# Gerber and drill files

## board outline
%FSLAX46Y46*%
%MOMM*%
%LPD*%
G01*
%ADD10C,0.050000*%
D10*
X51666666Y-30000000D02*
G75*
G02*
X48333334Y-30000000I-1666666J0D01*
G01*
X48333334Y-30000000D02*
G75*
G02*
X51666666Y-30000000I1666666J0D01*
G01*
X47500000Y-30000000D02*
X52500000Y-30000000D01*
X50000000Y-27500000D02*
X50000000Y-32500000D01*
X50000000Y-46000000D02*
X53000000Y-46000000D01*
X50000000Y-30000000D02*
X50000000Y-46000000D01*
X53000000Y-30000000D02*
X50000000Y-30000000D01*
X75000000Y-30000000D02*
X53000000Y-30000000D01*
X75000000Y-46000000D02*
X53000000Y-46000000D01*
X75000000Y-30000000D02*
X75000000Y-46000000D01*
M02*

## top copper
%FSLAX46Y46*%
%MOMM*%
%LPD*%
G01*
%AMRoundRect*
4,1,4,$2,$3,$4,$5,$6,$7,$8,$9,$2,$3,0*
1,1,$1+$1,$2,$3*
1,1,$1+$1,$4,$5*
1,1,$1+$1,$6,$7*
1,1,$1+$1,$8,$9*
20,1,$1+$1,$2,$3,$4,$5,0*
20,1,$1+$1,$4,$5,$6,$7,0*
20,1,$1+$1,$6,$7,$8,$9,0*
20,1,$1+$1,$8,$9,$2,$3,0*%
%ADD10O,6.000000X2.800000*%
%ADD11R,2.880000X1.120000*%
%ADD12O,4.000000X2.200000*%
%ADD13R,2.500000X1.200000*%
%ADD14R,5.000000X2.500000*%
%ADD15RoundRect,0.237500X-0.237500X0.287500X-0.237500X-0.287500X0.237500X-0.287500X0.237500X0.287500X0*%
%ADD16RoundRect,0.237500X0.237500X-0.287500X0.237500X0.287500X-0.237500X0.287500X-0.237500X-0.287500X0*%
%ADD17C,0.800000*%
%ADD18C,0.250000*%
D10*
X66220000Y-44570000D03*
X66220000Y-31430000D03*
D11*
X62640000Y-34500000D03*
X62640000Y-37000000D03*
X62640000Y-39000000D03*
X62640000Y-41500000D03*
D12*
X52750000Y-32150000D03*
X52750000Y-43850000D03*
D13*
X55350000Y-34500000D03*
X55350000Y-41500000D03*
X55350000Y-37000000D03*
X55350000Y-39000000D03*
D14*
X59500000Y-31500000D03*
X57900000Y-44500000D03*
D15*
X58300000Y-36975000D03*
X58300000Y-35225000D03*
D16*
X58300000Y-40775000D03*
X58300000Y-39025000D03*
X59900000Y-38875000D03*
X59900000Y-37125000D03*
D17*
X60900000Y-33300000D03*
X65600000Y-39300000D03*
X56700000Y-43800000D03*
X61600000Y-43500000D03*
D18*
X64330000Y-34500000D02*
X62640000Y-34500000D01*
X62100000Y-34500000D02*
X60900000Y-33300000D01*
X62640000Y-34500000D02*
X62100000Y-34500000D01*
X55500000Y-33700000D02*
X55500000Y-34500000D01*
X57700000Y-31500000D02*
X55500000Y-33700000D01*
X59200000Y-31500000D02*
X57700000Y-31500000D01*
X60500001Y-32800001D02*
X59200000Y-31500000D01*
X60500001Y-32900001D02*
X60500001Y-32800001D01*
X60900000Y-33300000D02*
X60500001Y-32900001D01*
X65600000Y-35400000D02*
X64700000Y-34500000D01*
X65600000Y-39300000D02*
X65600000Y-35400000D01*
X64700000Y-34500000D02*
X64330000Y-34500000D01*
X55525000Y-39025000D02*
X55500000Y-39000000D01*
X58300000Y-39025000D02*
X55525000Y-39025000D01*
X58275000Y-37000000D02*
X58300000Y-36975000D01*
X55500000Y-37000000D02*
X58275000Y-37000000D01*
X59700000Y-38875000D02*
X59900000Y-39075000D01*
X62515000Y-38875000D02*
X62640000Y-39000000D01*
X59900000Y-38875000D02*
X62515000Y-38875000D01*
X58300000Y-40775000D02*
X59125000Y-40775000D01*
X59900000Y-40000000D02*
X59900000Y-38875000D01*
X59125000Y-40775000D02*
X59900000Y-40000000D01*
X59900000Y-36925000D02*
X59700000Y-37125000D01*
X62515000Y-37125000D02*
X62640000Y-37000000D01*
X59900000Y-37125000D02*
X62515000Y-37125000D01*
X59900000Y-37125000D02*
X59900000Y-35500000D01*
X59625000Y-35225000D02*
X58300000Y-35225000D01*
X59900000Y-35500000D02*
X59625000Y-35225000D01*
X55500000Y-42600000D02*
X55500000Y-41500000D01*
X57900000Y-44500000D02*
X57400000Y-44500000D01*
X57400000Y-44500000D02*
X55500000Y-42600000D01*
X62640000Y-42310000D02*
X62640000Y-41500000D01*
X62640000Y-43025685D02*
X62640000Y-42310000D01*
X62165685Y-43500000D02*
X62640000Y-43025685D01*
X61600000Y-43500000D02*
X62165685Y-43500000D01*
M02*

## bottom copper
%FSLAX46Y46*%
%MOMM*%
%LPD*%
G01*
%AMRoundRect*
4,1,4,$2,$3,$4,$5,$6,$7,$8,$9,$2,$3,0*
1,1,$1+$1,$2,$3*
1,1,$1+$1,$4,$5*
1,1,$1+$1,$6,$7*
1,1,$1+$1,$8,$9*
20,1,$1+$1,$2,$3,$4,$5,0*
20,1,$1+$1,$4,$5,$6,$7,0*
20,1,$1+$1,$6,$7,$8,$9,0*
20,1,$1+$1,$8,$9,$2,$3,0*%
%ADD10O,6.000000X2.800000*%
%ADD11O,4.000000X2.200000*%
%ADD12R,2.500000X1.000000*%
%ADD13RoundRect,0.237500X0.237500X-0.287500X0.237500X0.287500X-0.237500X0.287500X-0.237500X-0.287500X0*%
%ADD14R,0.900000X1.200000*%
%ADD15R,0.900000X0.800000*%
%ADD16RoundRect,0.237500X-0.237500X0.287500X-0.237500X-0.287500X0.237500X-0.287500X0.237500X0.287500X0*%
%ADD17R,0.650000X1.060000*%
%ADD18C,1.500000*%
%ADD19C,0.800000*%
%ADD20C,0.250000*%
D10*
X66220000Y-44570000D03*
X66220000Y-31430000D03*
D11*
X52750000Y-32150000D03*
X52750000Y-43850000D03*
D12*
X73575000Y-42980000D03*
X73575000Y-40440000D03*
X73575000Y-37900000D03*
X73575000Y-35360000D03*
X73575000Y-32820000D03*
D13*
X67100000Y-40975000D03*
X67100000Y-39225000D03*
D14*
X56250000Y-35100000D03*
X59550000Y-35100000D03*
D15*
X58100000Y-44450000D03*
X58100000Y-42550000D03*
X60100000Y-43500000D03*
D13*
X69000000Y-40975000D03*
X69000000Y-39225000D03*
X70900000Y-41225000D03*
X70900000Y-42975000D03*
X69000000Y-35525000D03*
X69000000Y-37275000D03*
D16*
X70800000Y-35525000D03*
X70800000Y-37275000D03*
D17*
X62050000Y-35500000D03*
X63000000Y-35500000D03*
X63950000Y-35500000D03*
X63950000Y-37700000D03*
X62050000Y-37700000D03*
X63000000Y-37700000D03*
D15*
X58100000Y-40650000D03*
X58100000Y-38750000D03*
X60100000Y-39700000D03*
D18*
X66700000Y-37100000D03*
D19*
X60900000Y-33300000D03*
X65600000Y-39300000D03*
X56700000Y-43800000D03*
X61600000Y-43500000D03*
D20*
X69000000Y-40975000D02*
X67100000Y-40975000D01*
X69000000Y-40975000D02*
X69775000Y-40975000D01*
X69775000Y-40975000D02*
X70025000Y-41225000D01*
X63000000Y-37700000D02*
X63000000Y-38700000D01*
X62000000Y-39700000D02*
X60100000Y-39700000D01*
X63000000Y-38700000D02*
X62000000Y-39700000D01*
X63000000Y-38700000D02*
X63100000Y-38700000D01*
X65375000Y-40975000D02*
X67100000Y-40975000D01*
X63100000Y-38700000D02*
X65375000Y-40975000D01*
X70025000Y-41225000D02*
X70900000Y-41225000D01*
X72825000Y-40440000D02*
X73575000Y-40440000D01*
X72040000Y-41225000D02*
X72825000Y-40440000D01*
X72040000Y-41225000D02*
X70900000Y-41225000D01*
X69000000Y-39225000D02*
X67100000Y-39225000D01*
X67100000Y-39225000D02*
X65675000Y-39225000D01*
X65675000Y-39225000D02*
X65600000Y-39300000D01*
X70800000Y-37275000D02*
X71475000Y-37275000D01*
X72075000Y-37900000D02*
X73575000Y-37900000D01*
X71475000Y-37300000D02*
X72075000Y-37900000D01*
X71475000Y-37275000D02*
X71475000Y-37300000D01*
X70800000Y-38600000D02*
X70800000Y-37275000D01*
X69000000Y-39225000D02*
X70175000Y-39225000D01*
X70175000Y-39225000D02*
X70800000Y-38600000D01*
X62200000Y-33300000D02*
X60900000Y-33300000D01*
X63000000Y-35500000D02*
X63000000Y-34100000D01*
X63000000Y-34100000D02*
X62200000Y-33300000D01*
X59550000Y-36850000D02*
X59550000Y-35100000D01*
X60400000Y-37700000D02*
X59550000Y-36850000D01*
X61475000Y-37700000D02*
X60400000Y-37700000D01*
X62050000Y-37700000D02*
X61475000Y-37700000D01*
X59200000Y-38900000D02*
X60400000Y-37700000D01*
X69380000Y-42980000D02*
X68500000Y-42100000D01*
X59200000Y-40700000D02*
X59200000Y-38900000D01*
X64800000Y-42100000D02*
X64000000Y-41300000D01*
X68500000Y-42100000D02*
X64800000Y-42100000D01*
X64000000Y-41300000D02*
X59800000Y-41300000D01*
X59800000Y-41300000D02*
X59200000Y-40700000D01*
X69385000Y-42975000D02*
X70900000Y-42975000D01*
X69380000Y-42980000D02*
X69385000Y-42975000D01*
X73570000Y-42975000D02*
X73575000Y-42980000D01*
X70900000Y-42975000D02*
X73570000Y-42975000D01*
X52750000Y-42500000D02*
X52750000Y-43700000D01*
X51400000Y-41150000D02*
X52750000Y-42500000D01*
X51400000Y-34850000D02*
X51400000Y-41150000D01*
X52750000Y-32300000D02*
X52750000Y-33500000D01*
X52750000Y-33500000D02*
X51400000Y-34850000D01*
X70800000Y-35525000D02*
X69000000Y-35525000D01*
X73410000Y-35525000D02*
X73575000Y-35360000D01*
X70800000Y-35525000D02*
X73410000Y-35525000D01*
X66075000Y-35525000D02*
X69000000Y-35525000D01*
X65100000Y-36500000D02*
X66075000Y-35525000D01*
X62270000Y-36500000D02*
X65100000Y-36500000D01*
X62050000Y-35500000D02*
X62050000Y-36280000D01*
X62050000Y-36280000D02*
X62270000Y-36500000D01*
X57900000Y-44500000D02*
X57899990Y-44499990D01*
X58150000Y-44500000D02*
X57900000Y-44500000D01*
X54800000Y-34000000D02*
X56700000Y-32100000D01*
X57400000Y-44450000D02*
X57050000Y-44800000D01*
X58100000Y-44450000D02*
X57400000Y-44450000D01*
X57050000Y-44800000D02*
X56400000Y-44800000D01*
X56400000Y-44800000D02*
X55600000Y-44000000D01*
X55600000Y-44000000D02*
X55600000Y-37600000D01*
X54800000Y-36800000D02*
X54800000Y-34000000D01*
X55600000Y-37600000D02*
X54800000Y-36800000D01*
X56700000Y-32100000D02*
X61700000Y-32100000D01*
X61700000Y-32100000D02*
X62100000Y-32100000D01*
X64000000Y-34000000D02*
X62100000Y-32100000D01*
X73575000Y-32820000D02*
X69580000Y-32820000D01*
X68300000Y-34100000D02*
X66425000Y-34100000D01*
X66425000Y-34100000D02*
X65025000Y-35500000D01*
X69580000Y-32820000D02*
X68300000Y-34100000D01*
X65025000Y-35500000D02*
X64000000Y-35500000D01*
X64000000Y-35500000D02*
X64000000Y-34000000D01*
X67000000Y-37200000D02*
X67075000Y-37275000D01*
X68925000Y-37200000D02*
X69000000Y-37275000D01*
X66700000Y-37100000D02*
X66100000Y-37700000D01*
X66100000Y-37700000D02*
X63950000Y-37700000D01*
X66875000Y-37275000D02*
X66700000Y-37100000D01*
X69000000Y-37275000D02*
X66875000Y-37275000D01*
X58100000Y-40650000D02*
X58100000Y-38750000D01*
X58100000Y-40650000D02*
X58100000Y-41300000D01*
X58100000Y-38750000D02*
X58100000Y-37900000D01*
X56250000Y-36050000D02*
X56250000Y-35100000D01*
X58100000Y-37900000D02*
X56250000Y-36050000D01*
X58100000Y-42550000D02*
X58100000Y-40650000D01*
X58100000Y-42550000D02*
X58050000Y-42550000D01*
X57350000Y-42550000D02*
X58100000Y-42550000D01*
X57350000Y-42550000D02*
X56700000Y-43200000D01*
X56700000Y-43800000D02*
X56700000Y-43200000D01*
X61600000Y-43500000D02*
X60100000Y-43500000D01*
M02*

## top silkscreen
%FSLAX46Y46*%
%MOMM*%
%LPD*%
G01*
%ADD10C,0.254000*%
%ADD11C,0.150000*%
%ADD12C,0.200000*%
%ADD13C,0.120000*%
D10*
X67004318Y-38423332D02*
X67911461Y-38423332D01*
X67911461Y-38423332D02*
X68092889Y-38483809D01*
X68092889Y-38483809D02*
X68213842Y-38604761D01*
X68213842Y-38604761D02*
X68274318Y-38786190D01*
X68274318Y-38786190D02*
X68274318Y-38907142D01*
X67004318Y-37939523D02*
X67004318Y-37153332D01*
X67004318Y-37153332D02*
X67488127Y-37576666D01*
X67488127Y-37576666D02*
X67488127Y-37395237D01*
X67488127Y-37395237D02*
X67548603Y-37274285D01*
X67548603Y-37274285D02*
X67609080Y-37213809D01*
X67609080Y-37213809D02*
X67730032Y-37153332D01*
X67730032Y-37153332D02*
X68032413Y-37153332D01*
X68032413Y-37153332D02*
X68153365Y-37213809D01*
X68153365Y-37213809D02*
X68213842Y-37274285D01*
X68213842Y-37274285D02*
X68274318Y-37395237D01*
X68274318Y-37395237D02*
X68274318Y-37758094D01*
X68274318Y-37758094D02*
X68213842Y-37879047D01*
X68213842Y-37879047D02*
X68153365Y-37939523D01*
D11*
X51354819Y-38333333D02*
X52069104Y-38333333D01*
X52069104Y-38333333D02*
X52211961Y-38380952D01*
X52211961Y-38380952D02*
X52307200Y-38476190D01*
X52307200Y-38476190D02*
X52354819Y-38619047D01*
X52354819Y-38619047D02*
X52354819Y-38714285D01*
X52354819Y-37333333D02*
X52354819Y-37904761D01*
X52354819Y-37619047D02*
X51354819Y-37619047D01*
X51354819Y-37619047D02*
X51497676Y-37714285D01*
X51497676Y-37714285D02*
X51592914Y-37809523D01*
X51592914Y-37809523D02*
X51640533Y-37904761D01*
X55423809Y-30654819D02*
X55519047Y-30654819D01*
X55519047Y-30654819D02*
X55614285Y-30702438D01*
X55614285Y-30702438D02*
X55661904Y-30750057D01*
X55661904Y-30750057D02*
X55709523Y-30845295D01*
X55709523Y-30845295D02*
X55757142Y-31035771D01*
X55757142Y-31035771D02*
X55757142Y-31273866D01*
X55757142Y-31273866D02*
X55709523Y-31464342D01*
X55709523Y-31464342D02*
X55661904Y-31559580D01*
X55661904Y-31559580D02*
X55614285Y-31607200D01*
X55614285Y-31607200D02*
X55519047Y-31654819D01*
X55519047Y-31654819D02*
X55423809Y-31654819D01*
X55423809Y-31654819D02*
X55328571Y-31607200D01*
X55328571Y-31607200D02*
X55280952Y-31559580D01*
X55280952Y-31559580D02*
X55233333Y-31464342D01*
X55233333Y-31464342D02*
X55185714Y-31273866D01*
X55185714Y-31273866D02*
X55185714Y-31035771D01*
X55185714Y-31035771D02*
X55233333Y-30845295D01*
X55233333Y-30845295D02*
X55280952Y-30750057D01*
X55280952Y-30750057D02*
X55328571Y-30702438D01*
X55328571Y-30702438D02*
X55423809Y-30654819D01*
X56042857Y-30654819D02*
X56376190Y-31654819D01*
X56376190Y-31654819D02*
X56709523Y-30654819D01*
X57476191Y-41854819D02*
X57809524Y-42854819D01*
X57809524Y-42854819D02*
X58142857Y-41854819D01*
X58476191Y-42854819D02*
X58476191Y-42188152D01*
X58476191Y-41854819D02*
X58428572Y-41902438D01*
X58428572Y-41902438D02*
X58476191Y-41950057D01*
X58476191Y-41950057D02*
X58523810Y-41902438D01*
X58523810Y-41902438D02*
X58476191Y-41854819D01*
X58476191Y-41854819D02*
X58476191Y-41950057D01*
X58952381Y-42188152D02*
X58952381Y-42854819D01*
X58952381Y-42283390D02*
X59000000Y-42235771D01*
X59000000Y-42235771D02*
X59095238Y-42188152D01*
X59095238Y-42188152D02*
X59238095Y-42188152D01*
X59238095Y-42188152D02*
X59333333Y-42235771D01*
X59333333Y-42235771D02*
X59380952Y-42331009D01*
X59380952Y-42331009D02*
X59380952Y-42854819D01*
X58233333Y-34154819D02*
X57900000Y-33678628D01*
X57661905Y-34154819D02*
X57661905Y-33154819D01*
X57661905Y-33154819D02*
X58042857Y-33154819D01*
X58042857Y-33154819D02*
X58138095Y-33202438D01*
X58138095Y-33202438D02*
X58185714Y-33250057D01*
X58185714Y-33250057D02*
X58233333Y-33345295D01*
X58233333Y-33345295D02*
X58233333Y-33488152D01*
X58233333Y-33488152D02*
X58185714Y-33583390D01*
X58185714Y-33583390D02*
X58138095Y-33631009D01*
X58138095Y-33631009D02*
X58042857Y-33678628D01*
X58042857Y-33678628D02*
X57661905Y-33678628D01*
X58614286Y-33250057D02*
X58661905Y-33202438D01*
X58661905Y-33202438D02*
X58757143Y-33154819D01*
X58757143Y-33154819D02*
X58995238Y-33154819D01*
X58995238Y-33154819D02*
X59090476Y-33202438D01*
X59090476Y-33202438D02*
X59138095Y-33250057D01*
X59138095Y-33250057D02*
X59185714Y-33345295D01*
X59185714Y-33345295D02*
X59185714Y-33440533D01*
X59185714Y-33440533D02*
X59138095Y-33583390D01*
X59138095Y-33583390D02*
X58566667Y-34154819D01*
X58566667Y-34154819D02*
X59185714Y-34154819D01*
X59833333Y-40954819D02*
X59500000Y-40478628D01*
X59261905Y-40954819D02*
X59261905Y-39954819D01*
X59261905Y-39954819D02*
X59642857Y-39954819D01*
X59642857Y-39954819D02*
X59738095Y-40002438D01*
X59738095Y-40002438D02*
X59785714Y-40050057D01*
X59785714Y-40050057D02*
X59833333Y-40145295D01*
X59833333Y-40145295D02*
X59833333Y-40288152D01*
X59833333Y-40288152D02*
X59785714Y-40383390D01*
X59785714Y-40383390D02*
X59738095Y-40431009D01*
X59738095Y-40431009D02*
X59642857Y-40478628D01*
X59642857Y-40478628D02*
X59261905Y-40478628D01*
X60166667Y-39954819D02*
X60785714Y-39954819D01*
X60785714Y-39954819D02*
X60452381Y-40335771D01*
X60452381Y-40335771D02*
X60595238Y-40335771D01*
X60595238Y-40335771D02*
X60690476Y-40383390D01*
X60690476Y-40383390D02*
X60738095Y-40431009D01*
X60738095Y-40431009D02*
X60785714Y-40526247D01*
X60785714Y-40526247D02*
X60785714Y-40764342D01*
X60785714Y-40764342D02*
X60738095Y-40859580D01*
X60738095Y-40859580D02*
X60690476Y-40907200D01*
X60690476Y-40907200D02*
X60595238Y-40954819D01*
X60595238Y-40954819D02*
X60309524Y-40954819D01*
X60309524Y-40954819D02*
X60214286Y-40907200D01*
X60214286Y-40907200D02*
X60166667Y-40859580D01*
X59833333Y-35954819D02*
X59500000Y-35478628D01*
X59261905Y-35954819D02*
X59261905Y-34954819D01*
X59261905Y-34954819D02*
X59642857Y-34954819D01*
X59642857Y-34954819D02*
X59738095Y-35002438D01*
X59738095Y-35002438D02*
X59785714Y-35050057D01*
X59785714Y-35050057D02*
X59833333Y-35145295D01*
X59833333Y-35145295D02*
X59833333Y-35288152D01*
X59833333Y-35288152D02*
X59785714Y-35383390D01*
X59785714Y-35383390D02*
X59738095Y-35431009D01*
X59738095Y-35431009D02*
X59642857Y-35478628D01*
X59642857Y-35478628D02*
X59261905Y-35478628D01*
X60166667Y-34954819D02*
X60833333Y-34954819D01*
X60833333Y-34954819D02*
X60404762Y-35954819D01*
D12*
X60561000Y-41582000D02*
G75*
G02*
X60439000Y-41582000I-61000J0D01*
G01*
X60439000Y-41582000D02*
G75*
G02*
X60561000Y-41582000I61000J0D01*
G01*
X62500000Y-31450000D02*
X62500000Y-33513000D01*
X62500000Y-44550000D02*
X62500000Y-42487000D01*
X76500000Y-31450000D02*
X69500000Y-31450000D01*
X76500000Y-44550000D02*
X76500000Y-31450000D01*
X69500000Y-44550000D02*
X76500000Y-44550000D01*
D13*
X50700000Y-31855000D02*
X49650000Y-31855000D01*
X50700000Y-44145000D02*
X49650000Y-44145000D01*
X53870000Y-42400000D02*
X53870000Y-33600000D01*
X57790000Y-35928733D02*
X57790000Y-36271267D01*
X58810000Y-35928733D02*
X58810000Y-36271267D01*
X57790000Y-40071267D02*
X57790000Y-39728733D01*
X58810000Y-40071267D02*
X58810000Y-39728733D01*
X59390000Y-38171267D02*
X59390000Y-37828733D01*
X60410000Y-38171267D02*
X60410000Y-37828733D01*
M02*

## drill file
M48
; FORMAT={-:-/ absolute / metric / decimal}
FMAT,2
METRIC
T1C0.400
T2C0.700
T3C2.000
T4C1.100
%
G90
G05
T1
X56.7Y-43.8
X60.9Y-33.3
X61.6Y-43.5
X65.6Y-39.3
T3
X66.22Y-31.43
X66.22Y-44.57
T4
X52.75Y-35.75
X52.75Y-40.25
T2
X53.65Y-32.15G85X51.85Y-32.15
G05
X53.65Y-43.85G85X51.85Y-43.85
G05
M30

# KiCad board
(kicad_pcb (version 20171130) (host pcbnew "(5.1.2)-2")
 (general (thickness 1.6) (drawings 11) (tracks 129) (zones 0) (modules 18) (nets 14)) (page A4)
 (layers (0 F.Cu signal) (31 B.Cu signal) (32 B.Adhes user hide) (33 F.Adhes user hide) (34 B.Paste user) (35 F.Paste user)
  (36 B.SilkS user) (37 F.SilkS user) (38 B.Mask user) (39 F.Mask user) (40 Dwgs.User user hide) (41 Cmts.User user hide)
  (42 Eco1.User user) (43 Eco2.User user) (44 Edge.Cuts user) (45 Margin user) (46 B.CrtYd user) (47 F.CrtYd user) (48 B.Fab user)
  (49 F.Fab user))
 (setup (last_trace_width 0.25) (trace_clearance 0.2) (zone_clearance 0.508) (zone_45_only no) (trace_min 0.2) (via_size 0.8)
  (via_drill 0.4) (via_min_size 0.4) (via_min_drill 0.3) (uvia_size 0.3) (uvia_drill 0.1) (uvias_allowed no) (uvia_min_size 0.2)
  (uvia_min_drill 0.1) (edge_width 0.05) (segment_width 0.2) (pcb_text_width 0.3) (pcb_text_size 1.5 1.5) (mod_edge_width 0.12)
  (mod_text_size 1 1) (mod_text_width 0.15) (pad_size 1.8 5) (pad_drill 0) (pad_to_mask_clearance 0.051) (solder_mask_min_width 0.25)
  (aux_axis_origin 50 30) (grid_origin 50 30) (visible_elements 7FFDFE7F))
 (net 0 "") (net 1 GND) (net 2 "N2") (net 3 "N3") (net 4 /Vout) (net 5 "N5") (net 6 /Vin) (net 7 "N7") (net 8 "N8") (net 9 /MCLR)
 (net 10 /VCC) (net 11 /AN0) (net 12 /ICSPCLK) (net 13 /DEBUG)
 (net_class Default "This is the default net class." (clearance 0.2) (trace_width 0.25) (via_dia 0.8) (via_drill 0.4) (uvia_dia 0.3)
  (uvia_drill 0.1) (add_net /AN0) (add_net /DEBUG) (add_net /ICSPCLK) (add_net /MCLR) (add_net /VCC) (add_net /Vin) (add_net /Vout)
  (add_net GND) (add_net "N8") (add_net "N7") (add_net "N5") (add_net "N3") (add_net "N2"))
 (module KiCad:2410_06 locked (layer F.Cu) (at 76.5 38 90)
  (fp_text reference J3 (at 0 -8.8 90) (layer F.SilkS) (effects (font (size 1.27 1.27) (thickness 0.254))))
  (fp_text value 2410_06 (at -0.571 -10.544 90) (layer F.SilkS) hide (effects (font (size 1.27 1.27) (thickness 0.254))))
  (fp_circle (center -3.582 -16) (end -3.582 -15.939) (layer F.SilkS) (width 0.2))
  (fp_line (start 6.55 -14) (end 4.487 -14) (layer F.SilkS) (width 0.2))
  (fp_line (start -6.55 -14) (end -4.487 -14) (layer F.SilkS) (width 0.2))
  (fp_line (start 6.55 0) (end 6.55 -7) (layer F.SilkS) (width 0.2))
  (fp_line (start -6.55 0) (end 6.55 0) (layer F.SilkS) (width 0.2))
  (fp_line (start -6.55 -7) (end -6.55 0) (layer F.SilkS) (width 0.2))
  (pad 6 thru_hole oval (at -6.57 -10.28 90) (size 2.8 6) (drill 2) (layers *.Cu *.Mask))
  (pad 5 thru_hole oval (at 6.57 -10.28 90) (size 2.8 6) (drill 2) (layers *.Cu *.Mask))
  (pad 4 smd rect (at 3.5 -13.86 90) (size 1.12 2.88) (layers F.Cu F.Paste F.Mask) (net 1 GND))
  (pad 3 smd rect (at 1 -13.86 90) (size 1.12 2.88) (layers F.Cu F.Paste F.Mask) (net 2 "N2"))
  (pad 2 smd rect (at -1 -13.86 90) (size 1.12 2.88) (layers F.Cu F.Paste F.Mask) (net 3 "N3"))
  (pad 1 smd rect (at -3.5 -13.86 90) (size 1.12 2.88) (layers F.Cu F.Paste F.Mask) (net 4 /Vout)))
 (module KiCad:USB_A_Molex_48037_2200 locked (layer F.Cu) (at 45.85 38 180)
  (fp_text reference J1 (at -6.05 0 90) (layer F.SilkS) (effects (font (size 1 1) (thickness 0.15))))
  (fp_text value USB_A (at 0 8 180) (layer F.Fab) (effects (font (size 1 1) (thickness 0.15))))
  (fp_line (start -4.85 6.145) (end -3.8 6.145) (layer F.SilkS) (width 0.12))
  (fp_line (start -4.85 -6.145) (end -3.8 -6.145) (layer F.SilkS) (width 0.12))
  (fp_line (start -8.02 -4.4) (end -8.02 4.4) (layer F.SilkS) (width 0.12))
  (pad "" np_thru_hole circle (at -6.9 2.25 180) (size 1.1 1.1) (drill 1.1) (layers *.Cu *.Mask))
  (pad "" np_thru_hole circle (at -6.9 -2.25 180) (size 1.1 1.1) (drill 1.1) (layers *.Cu *.Mask))
  (pad 5 thru_hole oval (at -6.9 5.85 180) (size 4 2.2) (drill oval 2.5 0.7) (layers *.Cu *.Mask) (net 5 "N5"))
  (pad 5 thru_hole oval (at -6.9 -5.85 180) (size 4 2.2) (drill oval 2.5 0.7) (layers *.Cu *.Mask) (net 5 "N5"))
  (pad 4 smd rect (at -9.5 3.5 180) (size 2.5 1.2) (layers F.Cu F.Paste F.Mask) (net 1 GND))
  (pad 1 smd rect (at -9.5 -3.5 180) (size 2.5 1.2) (layers F.Cu F.Paste F.Mask) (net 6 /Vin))
  (pad 3 smd rect (at -9.5 1 180) (size 2.5 1.2) (layers F.Cu F.Paste F.Mask) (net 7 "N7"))
  (pad 2 smd rect (at -9.5 -1 180) (size 2.5 1.2) (layers F.Cu F.Paste F.Mask) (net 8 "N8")))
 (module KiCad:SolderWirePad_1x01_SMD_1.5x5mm (layer F.Cu) (at 59.5 31.5 90)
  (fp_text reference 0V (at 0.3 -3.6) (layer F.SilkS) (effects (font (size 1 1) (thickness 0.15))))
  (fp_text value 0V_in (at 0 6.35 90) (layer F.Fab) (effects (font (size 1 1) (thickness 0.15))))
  (pad 1 smd rect (at 0 0 90) (size 2.5 5) (layers F.Cu F.Paste F.Mask) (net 1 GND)))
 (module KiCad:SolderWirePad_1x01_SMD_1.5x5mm (layer F.Cu) (at 57.9 44.5 270)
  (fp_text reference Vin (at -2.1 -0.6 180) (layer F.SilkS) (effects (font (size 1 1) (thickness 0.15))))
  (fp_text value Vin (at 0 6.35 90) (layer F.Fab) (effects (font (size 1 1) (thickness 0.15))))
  (pad 1 smd rect (at 0 0 270) (size 2.5 5) (layers F.Cu F.Paste F.Mask) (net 6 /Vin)))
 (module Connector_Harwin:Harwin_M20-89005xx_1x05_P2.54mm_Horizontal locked (layer B.Cu) (at 79.1 37.9)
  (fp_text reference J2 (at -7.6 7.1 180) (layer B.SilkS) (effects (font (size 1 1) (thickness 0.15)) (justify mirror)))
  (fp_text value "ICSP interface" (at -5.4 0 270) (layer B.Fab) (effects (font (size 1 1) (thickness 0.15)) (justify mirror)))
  (pad 1 smd rect (at -5.525 5.08) (size 2.5 1) (layers B.Cu B.Paste B.Mask) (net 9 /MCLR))
  (pad 2 smd rect (at -5.525 2.54) (size 2.5 1) (layers B.Cu B.Paste B.Mask) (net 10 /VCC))
  (pad 3 smd rect (at -5.525 0) (size 2.5 1) (layers B.Cu B.Paste B.Mask) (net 1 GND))
  (pad 4 smd rect (at -5.525 -2.54) (size 2.5 1) (layers B.Cu B.Paste B.Mask) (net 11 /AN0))
  (pad 5 smd rect (at -5.525 -5.08) (size 2.5 1) (layers B.Cu B.Paste B.Mask) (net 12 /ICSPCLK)))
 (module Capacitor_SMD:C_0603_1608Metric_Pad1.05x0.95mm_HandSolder (layer B.Cu) (at 67.1 40.1 90)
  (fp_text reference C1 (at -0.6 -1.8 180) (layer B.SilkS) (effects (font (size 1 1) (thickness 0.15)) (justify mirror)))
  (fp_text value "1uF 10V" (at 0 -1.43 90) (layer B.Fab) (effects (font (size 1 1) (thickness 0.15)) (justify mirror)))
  (pad 1 smd roundrect (at -0.875 0 90) (size 1.05 0.95) (layers B.Cu B.Paste B.Mask) (roundrect_rratio 0.25) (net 10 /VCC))
  (pad 2 smd roundrect (at 0.875 0 90) (size 1.05 0.95) (layers B.Cu B.Paste B.Mask) (roundrect_rratio 0.25) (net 1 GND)))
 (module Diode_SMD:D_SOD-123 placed (layer B.Cu) (at 57.9 35.1)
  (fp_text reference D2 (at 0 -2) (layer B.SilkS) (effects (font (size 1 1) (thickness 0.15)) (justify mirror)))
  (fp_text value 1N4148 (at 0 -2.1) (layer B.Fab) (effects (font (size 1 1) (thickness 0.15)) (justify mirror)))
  (pad 1 smd rect (at -1.65 0) (size 0.9 1.2) (layers B.Cu B.Paste B.Mask) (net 6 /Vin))
  (pad 2 smd rect (at 1.65 0) (size 0.9 1.2) (layers B.Cu B.Paste B.Mask) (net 9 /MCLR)))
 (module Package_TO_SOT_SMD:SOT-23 (layer B.Cu) (at 59.1 43.5)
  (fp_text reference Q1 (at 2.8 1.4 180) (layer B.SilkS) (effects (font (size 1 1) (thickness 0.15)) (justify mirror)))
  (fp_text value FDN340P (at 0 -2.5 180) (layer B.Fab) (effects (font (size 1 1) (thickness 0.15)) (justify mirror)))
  (pad 1 smd rect (at -1 0.95) (size 0.9 0.8) (layers B.Cu B.Paste B.Mask) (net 12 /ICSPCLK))
  (pad 2 smd rect (at -1 -0.95) (size 0.9 0.8) (layers B.Cu B.Paste B.Mask) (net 6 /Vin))
  (pad 3 smd rect (at 1 0) (size 0.9 0.8) (layers B.Cu B.Paste B.Mask) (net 4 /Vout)))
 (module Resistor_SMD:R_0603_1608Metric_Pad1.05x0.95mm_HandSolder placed (layer B.Cu) (at 69 40.1 90)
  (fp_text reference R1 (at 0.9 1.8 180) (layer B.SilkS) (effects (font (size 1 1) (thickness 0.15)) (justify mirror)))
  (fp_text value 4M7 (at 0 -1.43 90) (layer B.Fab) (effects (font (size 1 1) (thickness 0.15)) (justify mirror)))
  (pad 1 smd roundrect (at -0.875 0 90) (size 1.05 0.95) (layers B.Cu B.Paste B.Mask) (roundrect_rratio 0.25) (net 10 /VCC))
  (pad 2 smd roundrect (at 0.875 0 90) (size 1.05 0.95) (layers B.Cu B.Paste B.Mask) (roundrect_rratio 0.25) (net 1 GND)))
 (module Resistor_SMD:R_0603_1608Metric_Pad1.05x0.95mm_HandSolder (layer F.Cu) (at 58.3 36.1 270)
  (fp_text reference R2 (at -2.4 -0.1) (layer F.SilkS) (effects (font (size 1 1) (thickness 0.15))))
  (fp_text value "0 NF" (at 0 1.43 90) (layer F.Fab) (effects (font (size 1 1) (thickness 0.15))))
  (fp_line (start -0.171267 0.51) (end 0.171267 0.51) (layer F.SilkS) (width 0.12))
  (fp_line (start -0.171267 -0.51) (end 0.171267 -0.51) (layer F.SilkS) (width 0.12))
  (pad 2 smd roundrect (at 0.875 0 270) (size 1.05 0.95) (layers F.Cu F.Paste F.Mask) (roundrect_rratio 0.25) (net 7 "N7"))
  (pad 1 smd roundrect (at -0.875 0 270) (size 1.05 0.95) (layers F.Cu F.Paste F.Mask) (roundrect_rratio 0.25) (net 2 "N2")))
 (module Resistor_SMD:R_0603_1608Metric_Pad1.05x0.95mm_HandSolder (layer F.Cu) (at 58.3 39.9 90)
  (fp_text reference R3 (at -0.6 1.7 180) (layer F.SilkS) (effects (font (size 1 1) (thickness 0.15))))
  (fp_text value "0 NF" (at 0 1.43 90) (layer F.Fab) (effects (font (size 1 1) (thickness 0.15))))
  (fp_line (start -0.171267 -0.51) (end 0.171267 -0.51) (layer F.SilkS) (width 0.12))
  (fp_line (start -0.171267 0.51) (end 0.171267 0.51) (layer F.SilkS) (width 0.12))
  (pad 1 smd roundrect (at -0.875 0 90) (size 1.05 0.95) (layers F.Cu F.Paste F.Mask) (roundrect_rratio 0.25) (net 3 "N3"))
  (pad 2 smd roundrect (at 0.875 0 90) (size 1.05 0.95) (layers F.Cu F.Paste F.Mask) (roundrect_rratio 0.25) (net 8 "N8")))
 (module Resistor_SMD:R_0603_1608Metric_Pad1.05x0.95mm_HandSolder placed (layer B.Cu) (at 70.9 42.1 90)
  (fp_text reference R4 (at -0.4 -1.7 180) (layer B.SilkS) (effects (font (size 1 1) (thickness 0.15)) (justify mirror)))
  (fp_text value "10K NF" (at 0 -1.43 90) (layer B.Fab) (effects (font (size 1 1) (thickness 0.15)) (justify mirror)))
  (pad 2 smd roundrect (at 0.875 0 90) (size 1.05 0.95) (layers B.Cu B.Paste B.Mask) (roundrect_rratio 0.25) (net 10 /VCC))
  (pad 1 smd roundrect (at -0.875 0 90) (size 1.05 0.95) (layers B.Cu B.Paste B.Mask) (roundrect_rratio 0.25) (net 9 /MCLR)))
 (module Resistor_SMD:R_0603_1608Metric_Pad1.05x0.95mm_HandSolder (layer B.Cu) (at 69 36.4 90)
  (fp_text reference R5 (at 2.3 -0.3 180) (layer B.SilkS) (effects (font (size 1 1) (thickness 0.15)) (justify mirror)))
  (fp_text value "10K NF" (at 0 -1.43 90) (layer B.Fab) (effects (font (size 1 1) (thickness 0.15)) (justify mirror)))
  (pad 2 smd roundrect (at 0.875 0 90) (size 1.05 0.95) (layers B.Cu B.Paste B.Mask) (roundrect_rratio 0.25) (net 11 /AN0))
  (pad 1 smd roundrect (at -0.875 0 90) (size 1.05 0.95) (layers B.Cu B.Paste B.Mask) (roundrect_rratio 0.25) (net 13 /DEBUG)))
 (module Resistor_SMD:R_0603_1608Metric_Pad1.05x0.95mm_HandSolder (layer B.Cu) (at 70.8 36.4 270)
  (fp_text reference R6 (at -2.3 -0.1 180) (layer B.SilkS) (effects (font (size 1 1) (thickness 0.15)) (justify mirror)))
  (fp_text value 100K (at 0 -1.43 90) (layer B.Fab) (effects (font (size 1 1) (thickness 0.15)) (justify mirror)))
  (pad 1 smd roundrect (at -0.875 0 270) (size 1.05 0.95) (layers B.Cu B.Paste B.Mask) (roundrect_rratio 0.25) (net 11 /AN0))
  (pad 2 smd roundrect (at 0.875 0 270) (size 1.05 0.95) (layers B.Cu B.Paste B.Mask) (roundrect_rratio 0.25) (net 1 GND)))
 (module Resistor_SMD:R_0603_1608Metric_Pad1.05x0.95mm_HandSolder (layer F.Cu) (at 59.9 38 90)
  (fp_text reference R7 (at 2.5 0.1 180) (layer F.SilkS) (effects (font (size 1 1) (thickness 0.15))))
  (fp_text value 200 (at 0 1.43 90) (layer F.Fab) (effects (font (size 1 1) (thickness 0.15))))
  (fp_line (start -0.171267 -0.51) (end 0.171267 -0.51) (layer F.SilkS) (width 0.12))
  (fp_line (start -0.171267 0.51) (end 0.171267 0.51) (layer F.SilkS) (width 0.12))
  (pad 1 smd roundrect (at -0.875 0 90) (size 1.05 0.95) (layers F.Cu F.Paste F.Mask) (roundrect_rratio 0.25) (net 3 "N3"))
  (pad 2 smd roundrect (at 0.875 0 90) (size 1.05 0.95) (layers F.Cu F.Paste F.Mask) (roundrect_rratio 0.25) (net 2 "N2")))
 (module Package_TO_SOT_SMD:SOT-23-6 (layer B.Cu) (at 63 36.6 270)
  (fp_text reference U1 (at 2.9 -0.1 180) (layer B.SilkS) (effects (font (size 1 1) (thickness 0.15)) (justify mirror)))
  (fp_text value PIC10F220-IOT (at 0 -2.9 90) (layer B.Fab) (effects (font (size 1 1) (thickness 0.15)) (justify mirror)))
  (pad 1 smd rect (at -1.1 0.95 270) (size 1.06 0.65) (layers B.Cu B.Paste B.Mask) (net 11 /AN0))
  (pad 2 smd rect (at -1.1 0 270) (size 1.06 0.65) (layers B.Cu B.Paste B.Mask) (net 1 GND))
  (pad 3 smd rect (at -1.1 -0.95 270) (size 1.06 0.65) (layers B.Cu B.Paste B.Mask) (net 12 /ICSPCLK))
  (pad 4 smd rect (at 1.1 -0.95 270) (size 1.06 0.65) (layers B.Cu B.Paste B.Mask) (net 13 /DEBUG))
  (pad 6 smd rect (at 1.1 0.95 270) (size 1.06 0.65) (layers B.Cu B.Paste B.Mask) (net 9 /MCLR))
  (pad 5 smd rect (at 1.1 0 270) (size 1.06 0.65) (layers B.Cu B.Paste B.Mask) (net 10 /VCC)))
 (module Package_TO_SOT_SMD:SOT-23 (layer B.Cu) (at 59.1 39.7)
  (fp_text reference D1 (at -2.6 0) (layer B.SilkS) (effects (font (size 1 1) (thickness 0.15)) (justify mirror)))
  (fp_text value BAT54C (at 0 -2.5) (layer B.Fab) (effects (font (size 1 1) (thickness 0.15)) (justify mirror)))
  (pad 1 smd rect (at -1 0.95) (size 0.9 0.8) (layers B.Cu B.Paste B.Mask) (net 6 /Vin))
  (pad 2 smd rect (at -1 -0.95) (size 0.9 0.8) (layers B.Cu B.Paste B.Mask) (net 6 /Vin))
  (pad 3 smd rect (at 1 0) (size 0.9 0.8) (layers B.Cu B.Paste B.Mask) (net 10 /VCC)))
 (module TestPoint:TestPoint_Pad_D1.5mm (layer B.Cu) (at 66.7 37.1)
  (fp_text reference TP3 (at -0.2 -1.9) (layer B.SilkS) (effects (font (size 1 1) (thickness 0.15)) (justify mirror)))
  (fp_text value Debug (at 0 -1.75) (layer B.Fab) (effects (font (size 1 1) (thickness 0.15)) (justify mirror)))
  (pad 1 smd circle (at 0 0) (size 1.5 1.5) (layers B.Cu B.Mask) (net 13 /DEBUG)))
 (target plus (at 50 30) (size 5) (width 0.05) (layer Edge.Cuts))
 (gr_line (start 50 46) (end 53 46) (layer Edge.Cuts) (width 0.05))
 (gr_line (start 50 30) (end 50 46) (layer Edge.Cuts) (width 0.05))
 (gr_line (start 53 30) (end 50 30) (layer Edge.Cuts) (width 0.05))
 (gr_line (start 75 30) (end 53 30) (layer Edge.Cuts) (width 0.05))
 (gr_line (start 75 46) (end 53 46) (layer Edge.Cuts) (width 0.05))
 (gr_line (start 75 30) (end 75 46) (layer Edge.Cuts) (width 0.05))
 (segment (start 69 40.975) (end 67.1 40.975) (width 0.25) (layer B.Cu) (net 10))
 (segment (start 69 40.975) (end 69.775 40.975) (width 0.25) (layer B.Cu) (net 10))
 (segment (start 69.775 40.975) (end 70.025 41.225) (width 0.25) (layer B.Cu) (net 10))
 (segment (start 63 37.7) (end 63 38.7) (width 0.25) (layer B.Cu) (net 10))
 (segment (start 62 39.7) (end 60.1 39.7) (width 0.25) (layer B.Cu) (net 10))
 (segment (start 63 38.7) (end 62 39.7) (width 0.25) (layer B.Cu) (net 10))
 (segment (start 63 38.7) (end 63.1 38.7) (width 0.25) (layer B.Cu) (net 10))
 (segment (start 65.375 40.975) (end 67.1 40.975) (width 0.25) (layer B.Cu) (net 10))
 (segment (start 63.1 38.7) (end 65.375 40.975) (width 0.25) (layer B.Cu) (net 10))
 (segment (start 70.025 41.225) (end 70.9 41.225) (width 0.25) (layer B.Cu) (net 10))
 (segment (start 72.825 40.44) (end 73.575 40.44) (width 0.25) (layer B.Cu) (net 10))
 (segment (start 72.04 41.225) (end 72.825 40.44) (width 0.25) (layer B.Cu) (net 10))
 (segment (start 72.04 41.225) (end 70.9 41.225) (width 0.25) (layer B.Cu) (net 10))
 (via (at 60.9 33.3) (size 0.8) (drill 0.4) (layers F.Cu B.Cu) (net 1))
 (segment (start 69 39.225) (end 67.1 39.225) (width 0.25) (layer B.Cu) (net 1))
 (segment (start 64.33 34.5) (end 62.64 34.5) (width 0.25) (layer F.Cu) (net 1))
 (segment (start 62.1 34.5) (end 60.9 33.3) (width 0.25) (layer F.Cu) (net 1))
 (segment (start 62.64 34.5) (end 62.1 34.5) (width 0.25) (layer F.Cu) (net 1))
 (segment (start 55.5 33.7) (end 55.5 34.5) (width 0.25) (layer F.Cu) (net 1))
 (segment (start 57.7 31.5) (end 55.5 33.7) (width 0.25) (layer F.Cu) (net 1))
 (segment (start 59.2 31.5) (end 57.7 31.5) (width 0.25) (layer F.Cu) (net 1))
 (segment (start 60.500001 32.800001) (end 59.2 31.5) (width 0.25) (layer F.Cu) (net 1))
 (segment (start 60.500001 32.900001) (end 60.500001 32.800001) (width 0.25) (layer F.Cu) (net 1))
 (segment (start 60.9 33.3) (end 60.500001 32.900001) (width 0.25) (layer F.Cu) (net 1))
 (via (at 65.6 39.3) (size 0.8) (drill 0.4) (layers F.Cu B.Cu) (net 1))
 (segment (start 67.1 39.225) (end 65.675 39.225) (width 0.25) (layer B.Cu) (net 1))
 (segment (start 65.675 39.225) (end 65.6 39.3) (width 0.25) (layer B.Cu) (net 1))
 (segment (start 65.6 35.4) (end 64.7 34.5) (width 0.25) (layer F.Cu) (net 1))
 (segment (start 65.6 39.3) (end 65.6 35.4) (width 0.25) (layer F.Cu) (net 1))
 (segment (start 64.7 34.5) (end 64.33 34.5) (width 0.25) (layer F.Cu) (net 1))
 (segment (start 70.8 37.275) (end 71.475 37.275) (width 0.25) (layer B.Cu) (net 1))
 (segment (start 72.075 37.9) (end 73.575 37.9) (width 0.25) (layer B.Cu) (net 1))
 (segment (start 71.475 37.3) (end 72.075 37.9) (width 0.25) (layer B.Cu) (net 1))
 (segment (start 71.475 37.275) (end 71.475 37.3) (width 0.25) (layer B.Cu) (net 1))
 (segment (start 70.8 38.6) (end 70.8 37.275) (width 0.25) (layer B.Cu) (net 1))
 (segment (start 69 39.225) (end 70.175 39.225) (width 0.25) (layer B.Cu) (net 1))
 (segment (start 70.175 39.225) (end 70.8 38.6) (width 0.25) (layer B.Cu) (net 1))
 (segment (start 62.2 33.3) (end 60.9 33.3) (width 0.25) (layer B.Cu) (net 1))
 (segment (start 63 35.5) (end 63 34.1) (width 0.25) (layer B.Cu) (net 1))
 (segment (start 63 34.1) (end 62.2 33.3) (width 0.25) (layer B.Cu) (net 1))
 (segment (start 59.55 36.85) (end 59.55 35.1) (width 0.25) (layer B.Cu) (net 9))
 (segment (start 60.4 37.7) (end 59.55 36.85) (width 0.25) (layer B.Cu) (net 9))
 (segment (start 61.475 37.7) (end 60.4 37.7) (width 0.25) (layer B.Cu) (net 9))
 (segment (start 62.05 37.7) (end 61.475 37.7) (width 0.25) (layer B.Cu) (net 9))
 (segment (start 59.2 38.9) (end 60.4 37.7) (width 0.25) (layer B.Cu) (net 9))
 (segment (start 69.38 42.98) (end 68.5 42.1) (width 0.25) (layer B.Cu) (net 9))
 (segment (start 59.2 40.7) (end 59.2 38.9) (width 0.25) (layer B.Cu) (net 9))
 (segment (start 64.8 42.1) (end 64 41.3) (width 0.25) (layer B.Cu) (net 9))
 (segment (start 68.5 42.1) (end 64.8 42.1) (width 0.25) (layer B.Cu) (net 9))
 (segment (start 64 41.3) (end 59.8 41.3) (width 0.25) (layer B.Cu) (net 9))
 (segment (start 59.8 41.3) (end 59.2 40.7) (width 0.25) (layer B.Cu) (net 9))
 (segment (start 69.385 42.975) (end 70.9 42.975) (width 0.25) (layer B.Cu) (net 9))
 (segment (start 69.38 42.98) (end 69.385 42.975) (width 0.25) (layer B.Cu) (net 9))
 (segment (start 73.57 42.975) (end 73.575 42.98) (width 0.25) (layer B.Cu) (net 9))
 (segment (start 70.9 42.975) (end 73.57 42.975) (width 0.25) (layer B.Cu) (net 9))
 (segment (start 55.525 39.025) (end 55.5 39) (width 0.25) (layer F.Cu) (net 8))
 (segment (start 58.3 39.025) (end 55.525 39.025) (width 0.25) (layer F.Cu) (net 8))
 (segment (start 58.275 37) (end 58.3 36.975) (width 0.25) (layer F.Cu) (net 7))
 (segment (start 55.5 37) (end 58.275 37) (width 0.25) (layer F.Cu) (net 7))
 (segment (start 52.75 42.5) (end 52.75 43.7) (width 0.25) (layer B.Cu) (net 5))
 (segment (start 51.4 41.15) (end 52.75 42.5) (width 0.25) (layer B.Cu) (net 5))
 (segment (start 51.4 34.85) (end 51.4 41.15) (width 0.25) (layer B.Cu) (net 5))
 (segment (start 52.75 32.3) (end 52.75 33.5) (width 0.25) (layer B.Cu) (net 5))
 (segment (start 52.75 33.5) (end 51.4 34.85) (width 0.25) (layer B.Cu) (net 5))
 (segment (start 70.8 35.525) (end 69 35.525) (width 0.25) (layer B.Cu) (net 11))
 (segment (start 73.41 35.525) (end 73.575 35.36) (width 0.25) (layer B.Cu) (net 11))
 (segment (start 70.8 35.525) (end 73.41 35.525) (width 0.25) (layer B.Cu) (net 11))
 (segment (start 66.075 35.525) (end 69 35.525) (width 0.25) (layer B.Cu) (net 11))
 (segment (start 65.1 36.5) (end 66.075 35.525) (width 0.25) (layer B.Cu) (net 11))
 (segment (start 62.27 36.5) (end 65.1 36.5) (width 0.25) (layer B.Cu) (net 11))
 (segment (start 62.05 35.5) (end 62.05 36.28) (width 0.25) (layer B.Cu) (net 11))
 (segment (start 62.05 36.28) (end 62.27 36.5) (width 0.25) (layer B.Cu) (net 11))
 (segment (start 57.9 44.5) (end 57.89999 44.49999) (width 0.25) (layer B.Cu) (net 12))
 (segment (start 58.15 44.5) (end 57.9 44.5) (width 0.25) (layer B.Cu) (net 12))
 (segment (start 54.8 34) (end 56.7 32.1) (width 0.25) (layer B.Cu) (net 12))
 (segment (start 57.4 44.45) (end 57.05 44.8) (width 0.25) (layer B.Cu) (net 12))
 (segment (start 58.1 44.45) (end 57.4 44.45) (width 0.25) (layer B.Cu) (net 12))
 (segment (start 57.05 44.8) (end 56.4 44.8) (width 0.25) (layer B.Cu) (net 12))
 (segment (start 56.4 44.8) (end 55.6 44) (width 0.25) (layer B.Cu) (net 12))
 (segment (start 55.6 44) (end 55.6 37.6) (width 0.25) (layer B.Cu) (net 12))
 (segment (start 54.8 36.8) (end 54.8 34) (width 0.25) (layer B.Cu) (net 12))
 (segment (start 55.6 37.6) (end 54.8 36.8) (width 0.25) (layer B.Cu) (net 12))
 (segment (start 56.7 32.1) (end 61.7 32.1) (width 0.25) (layer B.Cu) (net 12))
 (segment (start 61.7 32.1) (end 62.1 32.1) (width 0.25) (layer B.Cu) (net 12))
 (segment (start 64 34) (end 62.1 32.1) (width 0.25) (layer B.Cu) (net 12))
 (segment (start 73.575 32.82) (end 69.58 32.82) (width 0.25) (layer B.Cu) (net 12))
 (segment (start 68.3 34.1) (end 66.425 34.1) (width 0.25) (layer B.Cu) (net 12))
 (segment (start 66.425 34.1) (end 65.025 35.5) (width 0.25) (layer B.Cu) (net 12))
 (segment (start 69.58 32.82) (end 68.3 34.1) (width 0.25) (layer B.Cu) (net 12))
 (segment (start 65.025 35.5) (end 64 35.5) (width 0.25) (layer B.Cu) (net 12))
 (segment (start 64 35.5) (end 64 34) (width 0.25) (layer B.Cu) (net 12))
 (segment (start 59.7 38.875) (end 59.9 39.075) (width 0.25) (layer F.Cu) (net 3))
 (segment (start 62.515 38.875) (end 62.64 39) (width 0.25) (layer F.Cu) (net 3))
 (segment (start 59.9 38.875) (end 62.515 38.875) (width 0.25) (layer F.Cu) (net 3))
 (segment (start 58.3 40.775) (end 59.125 40.775) (width 0.25) (layer F.Cu) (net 3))
 (segment (start 59.9 40) (end 59.9 38.875) (width 0.25) (layer F.Cu) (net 3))
 (segment (start 59.125 40.775) (end 59.9 40) (width 0.25) (layer F.Cu) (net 3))
 (segment (start 59.9 36.925) (end 59.7 37.125) (width 0.25) (layer F.Cu) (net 2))
 (segment (start 62.515 37.125) (end 62.64 37) (width 0.25) (layer F.Cu) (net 2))
 (segment (start 59.9 37.125) (end 62.515 37.125) (width 0.25) (layer F.Cu) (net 2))
 (segment (start 59.9 37.125) (end 59.9 35.5) (width 0.25) (layer F.Cu) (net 2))
 (segment (start 59.625 35.225) (end 58.3 35.225) (width 0.25) (layer F.Cu) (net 2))
 (segment (start 59.9 35.5) (end 59.625 35.225) (width 0.25) (layer F.Cu) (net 2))
 (segment (start 67 37.2) (end 67.075 37.275) (width 0.25) (layer B.Cu) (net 13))
 (segment (start 68.925 37.2) (end 69 37.275) (width 0.25) (layer B.Cu) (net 13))
 (segment (start 66.7 37.1) (end 66.1 37.7) (width 0.25) (layer B.Cu) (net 13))
 (segment (start 66.1 37.7) (end 63.95 37.7) (width 0.25) (layer B.Cu) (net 13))
 (segment (start 66.875 37.275) (end 66.7 37.1) (width 0.25) (layer B.Cu) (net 13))
 (segment (start 69 37.275) (end 66.875 37.275) (width 0.25) (layer B.Cu) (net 13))
 (segment (start 58.1 40.65) (end 58.1 38.75) (width 0.25) (layer B.Cu) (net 6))
 (segment (start 58.1 40.65) (end 58.1 41.3) (width 0.25) (layer B.Cu) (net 6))
 (segment (start 58.1 38.75) (end 58.1 37.9) (width 0.25) (layer B.Cu) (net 6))
 (segment (start 56.25 36.05) (end 56.25 35.1) (width 0.25) (layer B.Cu) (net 6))
 (segment (start 58.1 37.9) (end 56.25 36.05) (width 0.25) (layer B.Cu) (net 6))
 (segment (start 58.1 42.55) (end 58.1 40.65) (width 0.25) (layer B.Cu) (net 6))
 (via (at 56.7 43.8) (size 0.8) (drill 0.4) (layers F.Cu B.Cu) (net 6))
 (segment (start 58.1 42.55) (end 58.05 42.55) (width 0.25) (layer B.Cu) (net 6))
 (segment (start 57.35 42.55) (end 58.1 42.55) (width 0.25) (layer B.Cu) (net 6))
 (segment (start 57.35 42.55) (end 56.7 43.2) (width 0.25) (layer B.Cu) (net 6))
 (segment (start 55.5 42.6) (end 55.5 41.5) (width 0.25) (layer F.Cu) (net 6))
 (segment (start 57.9 44.5) (end 57.4 44.5) (width 0.25) (layer F.Cu) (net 6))
 (segment (start 57.4 44.5) (end 55.5 42.6) (width 0.25) (layer F.Cu) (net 6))
 (segment (start 56.7 43.8) (end 56.7 43.2) (width 0.25) (layer B.Cu) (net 6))
 (via (at 61.6 43.5) (size 0.8) (drill 0.4) (layers F.Cu B.Cu) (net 4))
 (segment (start 61.6 43.5) (end 60.1 43.5) (width 0.25) (layer B.Cu) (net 4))
 (segment (start 62.64 42.31) (end 62.64 41.5) (width 0.25) (layer F.Cu) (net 4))
 (segment (start 62.64 43.025685) (end 62.64 42.31) (width 0.25) (layer F.Cu) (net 4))
 (segment (start 62.165685 43.5) (end 62.64 43.025685) (width 0.25) (layer F.Cu) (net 4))
 (segment (start 61.6 43.5) (end 62.165685 43.5) (width 0.25) (layer F.Cu) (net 4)))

